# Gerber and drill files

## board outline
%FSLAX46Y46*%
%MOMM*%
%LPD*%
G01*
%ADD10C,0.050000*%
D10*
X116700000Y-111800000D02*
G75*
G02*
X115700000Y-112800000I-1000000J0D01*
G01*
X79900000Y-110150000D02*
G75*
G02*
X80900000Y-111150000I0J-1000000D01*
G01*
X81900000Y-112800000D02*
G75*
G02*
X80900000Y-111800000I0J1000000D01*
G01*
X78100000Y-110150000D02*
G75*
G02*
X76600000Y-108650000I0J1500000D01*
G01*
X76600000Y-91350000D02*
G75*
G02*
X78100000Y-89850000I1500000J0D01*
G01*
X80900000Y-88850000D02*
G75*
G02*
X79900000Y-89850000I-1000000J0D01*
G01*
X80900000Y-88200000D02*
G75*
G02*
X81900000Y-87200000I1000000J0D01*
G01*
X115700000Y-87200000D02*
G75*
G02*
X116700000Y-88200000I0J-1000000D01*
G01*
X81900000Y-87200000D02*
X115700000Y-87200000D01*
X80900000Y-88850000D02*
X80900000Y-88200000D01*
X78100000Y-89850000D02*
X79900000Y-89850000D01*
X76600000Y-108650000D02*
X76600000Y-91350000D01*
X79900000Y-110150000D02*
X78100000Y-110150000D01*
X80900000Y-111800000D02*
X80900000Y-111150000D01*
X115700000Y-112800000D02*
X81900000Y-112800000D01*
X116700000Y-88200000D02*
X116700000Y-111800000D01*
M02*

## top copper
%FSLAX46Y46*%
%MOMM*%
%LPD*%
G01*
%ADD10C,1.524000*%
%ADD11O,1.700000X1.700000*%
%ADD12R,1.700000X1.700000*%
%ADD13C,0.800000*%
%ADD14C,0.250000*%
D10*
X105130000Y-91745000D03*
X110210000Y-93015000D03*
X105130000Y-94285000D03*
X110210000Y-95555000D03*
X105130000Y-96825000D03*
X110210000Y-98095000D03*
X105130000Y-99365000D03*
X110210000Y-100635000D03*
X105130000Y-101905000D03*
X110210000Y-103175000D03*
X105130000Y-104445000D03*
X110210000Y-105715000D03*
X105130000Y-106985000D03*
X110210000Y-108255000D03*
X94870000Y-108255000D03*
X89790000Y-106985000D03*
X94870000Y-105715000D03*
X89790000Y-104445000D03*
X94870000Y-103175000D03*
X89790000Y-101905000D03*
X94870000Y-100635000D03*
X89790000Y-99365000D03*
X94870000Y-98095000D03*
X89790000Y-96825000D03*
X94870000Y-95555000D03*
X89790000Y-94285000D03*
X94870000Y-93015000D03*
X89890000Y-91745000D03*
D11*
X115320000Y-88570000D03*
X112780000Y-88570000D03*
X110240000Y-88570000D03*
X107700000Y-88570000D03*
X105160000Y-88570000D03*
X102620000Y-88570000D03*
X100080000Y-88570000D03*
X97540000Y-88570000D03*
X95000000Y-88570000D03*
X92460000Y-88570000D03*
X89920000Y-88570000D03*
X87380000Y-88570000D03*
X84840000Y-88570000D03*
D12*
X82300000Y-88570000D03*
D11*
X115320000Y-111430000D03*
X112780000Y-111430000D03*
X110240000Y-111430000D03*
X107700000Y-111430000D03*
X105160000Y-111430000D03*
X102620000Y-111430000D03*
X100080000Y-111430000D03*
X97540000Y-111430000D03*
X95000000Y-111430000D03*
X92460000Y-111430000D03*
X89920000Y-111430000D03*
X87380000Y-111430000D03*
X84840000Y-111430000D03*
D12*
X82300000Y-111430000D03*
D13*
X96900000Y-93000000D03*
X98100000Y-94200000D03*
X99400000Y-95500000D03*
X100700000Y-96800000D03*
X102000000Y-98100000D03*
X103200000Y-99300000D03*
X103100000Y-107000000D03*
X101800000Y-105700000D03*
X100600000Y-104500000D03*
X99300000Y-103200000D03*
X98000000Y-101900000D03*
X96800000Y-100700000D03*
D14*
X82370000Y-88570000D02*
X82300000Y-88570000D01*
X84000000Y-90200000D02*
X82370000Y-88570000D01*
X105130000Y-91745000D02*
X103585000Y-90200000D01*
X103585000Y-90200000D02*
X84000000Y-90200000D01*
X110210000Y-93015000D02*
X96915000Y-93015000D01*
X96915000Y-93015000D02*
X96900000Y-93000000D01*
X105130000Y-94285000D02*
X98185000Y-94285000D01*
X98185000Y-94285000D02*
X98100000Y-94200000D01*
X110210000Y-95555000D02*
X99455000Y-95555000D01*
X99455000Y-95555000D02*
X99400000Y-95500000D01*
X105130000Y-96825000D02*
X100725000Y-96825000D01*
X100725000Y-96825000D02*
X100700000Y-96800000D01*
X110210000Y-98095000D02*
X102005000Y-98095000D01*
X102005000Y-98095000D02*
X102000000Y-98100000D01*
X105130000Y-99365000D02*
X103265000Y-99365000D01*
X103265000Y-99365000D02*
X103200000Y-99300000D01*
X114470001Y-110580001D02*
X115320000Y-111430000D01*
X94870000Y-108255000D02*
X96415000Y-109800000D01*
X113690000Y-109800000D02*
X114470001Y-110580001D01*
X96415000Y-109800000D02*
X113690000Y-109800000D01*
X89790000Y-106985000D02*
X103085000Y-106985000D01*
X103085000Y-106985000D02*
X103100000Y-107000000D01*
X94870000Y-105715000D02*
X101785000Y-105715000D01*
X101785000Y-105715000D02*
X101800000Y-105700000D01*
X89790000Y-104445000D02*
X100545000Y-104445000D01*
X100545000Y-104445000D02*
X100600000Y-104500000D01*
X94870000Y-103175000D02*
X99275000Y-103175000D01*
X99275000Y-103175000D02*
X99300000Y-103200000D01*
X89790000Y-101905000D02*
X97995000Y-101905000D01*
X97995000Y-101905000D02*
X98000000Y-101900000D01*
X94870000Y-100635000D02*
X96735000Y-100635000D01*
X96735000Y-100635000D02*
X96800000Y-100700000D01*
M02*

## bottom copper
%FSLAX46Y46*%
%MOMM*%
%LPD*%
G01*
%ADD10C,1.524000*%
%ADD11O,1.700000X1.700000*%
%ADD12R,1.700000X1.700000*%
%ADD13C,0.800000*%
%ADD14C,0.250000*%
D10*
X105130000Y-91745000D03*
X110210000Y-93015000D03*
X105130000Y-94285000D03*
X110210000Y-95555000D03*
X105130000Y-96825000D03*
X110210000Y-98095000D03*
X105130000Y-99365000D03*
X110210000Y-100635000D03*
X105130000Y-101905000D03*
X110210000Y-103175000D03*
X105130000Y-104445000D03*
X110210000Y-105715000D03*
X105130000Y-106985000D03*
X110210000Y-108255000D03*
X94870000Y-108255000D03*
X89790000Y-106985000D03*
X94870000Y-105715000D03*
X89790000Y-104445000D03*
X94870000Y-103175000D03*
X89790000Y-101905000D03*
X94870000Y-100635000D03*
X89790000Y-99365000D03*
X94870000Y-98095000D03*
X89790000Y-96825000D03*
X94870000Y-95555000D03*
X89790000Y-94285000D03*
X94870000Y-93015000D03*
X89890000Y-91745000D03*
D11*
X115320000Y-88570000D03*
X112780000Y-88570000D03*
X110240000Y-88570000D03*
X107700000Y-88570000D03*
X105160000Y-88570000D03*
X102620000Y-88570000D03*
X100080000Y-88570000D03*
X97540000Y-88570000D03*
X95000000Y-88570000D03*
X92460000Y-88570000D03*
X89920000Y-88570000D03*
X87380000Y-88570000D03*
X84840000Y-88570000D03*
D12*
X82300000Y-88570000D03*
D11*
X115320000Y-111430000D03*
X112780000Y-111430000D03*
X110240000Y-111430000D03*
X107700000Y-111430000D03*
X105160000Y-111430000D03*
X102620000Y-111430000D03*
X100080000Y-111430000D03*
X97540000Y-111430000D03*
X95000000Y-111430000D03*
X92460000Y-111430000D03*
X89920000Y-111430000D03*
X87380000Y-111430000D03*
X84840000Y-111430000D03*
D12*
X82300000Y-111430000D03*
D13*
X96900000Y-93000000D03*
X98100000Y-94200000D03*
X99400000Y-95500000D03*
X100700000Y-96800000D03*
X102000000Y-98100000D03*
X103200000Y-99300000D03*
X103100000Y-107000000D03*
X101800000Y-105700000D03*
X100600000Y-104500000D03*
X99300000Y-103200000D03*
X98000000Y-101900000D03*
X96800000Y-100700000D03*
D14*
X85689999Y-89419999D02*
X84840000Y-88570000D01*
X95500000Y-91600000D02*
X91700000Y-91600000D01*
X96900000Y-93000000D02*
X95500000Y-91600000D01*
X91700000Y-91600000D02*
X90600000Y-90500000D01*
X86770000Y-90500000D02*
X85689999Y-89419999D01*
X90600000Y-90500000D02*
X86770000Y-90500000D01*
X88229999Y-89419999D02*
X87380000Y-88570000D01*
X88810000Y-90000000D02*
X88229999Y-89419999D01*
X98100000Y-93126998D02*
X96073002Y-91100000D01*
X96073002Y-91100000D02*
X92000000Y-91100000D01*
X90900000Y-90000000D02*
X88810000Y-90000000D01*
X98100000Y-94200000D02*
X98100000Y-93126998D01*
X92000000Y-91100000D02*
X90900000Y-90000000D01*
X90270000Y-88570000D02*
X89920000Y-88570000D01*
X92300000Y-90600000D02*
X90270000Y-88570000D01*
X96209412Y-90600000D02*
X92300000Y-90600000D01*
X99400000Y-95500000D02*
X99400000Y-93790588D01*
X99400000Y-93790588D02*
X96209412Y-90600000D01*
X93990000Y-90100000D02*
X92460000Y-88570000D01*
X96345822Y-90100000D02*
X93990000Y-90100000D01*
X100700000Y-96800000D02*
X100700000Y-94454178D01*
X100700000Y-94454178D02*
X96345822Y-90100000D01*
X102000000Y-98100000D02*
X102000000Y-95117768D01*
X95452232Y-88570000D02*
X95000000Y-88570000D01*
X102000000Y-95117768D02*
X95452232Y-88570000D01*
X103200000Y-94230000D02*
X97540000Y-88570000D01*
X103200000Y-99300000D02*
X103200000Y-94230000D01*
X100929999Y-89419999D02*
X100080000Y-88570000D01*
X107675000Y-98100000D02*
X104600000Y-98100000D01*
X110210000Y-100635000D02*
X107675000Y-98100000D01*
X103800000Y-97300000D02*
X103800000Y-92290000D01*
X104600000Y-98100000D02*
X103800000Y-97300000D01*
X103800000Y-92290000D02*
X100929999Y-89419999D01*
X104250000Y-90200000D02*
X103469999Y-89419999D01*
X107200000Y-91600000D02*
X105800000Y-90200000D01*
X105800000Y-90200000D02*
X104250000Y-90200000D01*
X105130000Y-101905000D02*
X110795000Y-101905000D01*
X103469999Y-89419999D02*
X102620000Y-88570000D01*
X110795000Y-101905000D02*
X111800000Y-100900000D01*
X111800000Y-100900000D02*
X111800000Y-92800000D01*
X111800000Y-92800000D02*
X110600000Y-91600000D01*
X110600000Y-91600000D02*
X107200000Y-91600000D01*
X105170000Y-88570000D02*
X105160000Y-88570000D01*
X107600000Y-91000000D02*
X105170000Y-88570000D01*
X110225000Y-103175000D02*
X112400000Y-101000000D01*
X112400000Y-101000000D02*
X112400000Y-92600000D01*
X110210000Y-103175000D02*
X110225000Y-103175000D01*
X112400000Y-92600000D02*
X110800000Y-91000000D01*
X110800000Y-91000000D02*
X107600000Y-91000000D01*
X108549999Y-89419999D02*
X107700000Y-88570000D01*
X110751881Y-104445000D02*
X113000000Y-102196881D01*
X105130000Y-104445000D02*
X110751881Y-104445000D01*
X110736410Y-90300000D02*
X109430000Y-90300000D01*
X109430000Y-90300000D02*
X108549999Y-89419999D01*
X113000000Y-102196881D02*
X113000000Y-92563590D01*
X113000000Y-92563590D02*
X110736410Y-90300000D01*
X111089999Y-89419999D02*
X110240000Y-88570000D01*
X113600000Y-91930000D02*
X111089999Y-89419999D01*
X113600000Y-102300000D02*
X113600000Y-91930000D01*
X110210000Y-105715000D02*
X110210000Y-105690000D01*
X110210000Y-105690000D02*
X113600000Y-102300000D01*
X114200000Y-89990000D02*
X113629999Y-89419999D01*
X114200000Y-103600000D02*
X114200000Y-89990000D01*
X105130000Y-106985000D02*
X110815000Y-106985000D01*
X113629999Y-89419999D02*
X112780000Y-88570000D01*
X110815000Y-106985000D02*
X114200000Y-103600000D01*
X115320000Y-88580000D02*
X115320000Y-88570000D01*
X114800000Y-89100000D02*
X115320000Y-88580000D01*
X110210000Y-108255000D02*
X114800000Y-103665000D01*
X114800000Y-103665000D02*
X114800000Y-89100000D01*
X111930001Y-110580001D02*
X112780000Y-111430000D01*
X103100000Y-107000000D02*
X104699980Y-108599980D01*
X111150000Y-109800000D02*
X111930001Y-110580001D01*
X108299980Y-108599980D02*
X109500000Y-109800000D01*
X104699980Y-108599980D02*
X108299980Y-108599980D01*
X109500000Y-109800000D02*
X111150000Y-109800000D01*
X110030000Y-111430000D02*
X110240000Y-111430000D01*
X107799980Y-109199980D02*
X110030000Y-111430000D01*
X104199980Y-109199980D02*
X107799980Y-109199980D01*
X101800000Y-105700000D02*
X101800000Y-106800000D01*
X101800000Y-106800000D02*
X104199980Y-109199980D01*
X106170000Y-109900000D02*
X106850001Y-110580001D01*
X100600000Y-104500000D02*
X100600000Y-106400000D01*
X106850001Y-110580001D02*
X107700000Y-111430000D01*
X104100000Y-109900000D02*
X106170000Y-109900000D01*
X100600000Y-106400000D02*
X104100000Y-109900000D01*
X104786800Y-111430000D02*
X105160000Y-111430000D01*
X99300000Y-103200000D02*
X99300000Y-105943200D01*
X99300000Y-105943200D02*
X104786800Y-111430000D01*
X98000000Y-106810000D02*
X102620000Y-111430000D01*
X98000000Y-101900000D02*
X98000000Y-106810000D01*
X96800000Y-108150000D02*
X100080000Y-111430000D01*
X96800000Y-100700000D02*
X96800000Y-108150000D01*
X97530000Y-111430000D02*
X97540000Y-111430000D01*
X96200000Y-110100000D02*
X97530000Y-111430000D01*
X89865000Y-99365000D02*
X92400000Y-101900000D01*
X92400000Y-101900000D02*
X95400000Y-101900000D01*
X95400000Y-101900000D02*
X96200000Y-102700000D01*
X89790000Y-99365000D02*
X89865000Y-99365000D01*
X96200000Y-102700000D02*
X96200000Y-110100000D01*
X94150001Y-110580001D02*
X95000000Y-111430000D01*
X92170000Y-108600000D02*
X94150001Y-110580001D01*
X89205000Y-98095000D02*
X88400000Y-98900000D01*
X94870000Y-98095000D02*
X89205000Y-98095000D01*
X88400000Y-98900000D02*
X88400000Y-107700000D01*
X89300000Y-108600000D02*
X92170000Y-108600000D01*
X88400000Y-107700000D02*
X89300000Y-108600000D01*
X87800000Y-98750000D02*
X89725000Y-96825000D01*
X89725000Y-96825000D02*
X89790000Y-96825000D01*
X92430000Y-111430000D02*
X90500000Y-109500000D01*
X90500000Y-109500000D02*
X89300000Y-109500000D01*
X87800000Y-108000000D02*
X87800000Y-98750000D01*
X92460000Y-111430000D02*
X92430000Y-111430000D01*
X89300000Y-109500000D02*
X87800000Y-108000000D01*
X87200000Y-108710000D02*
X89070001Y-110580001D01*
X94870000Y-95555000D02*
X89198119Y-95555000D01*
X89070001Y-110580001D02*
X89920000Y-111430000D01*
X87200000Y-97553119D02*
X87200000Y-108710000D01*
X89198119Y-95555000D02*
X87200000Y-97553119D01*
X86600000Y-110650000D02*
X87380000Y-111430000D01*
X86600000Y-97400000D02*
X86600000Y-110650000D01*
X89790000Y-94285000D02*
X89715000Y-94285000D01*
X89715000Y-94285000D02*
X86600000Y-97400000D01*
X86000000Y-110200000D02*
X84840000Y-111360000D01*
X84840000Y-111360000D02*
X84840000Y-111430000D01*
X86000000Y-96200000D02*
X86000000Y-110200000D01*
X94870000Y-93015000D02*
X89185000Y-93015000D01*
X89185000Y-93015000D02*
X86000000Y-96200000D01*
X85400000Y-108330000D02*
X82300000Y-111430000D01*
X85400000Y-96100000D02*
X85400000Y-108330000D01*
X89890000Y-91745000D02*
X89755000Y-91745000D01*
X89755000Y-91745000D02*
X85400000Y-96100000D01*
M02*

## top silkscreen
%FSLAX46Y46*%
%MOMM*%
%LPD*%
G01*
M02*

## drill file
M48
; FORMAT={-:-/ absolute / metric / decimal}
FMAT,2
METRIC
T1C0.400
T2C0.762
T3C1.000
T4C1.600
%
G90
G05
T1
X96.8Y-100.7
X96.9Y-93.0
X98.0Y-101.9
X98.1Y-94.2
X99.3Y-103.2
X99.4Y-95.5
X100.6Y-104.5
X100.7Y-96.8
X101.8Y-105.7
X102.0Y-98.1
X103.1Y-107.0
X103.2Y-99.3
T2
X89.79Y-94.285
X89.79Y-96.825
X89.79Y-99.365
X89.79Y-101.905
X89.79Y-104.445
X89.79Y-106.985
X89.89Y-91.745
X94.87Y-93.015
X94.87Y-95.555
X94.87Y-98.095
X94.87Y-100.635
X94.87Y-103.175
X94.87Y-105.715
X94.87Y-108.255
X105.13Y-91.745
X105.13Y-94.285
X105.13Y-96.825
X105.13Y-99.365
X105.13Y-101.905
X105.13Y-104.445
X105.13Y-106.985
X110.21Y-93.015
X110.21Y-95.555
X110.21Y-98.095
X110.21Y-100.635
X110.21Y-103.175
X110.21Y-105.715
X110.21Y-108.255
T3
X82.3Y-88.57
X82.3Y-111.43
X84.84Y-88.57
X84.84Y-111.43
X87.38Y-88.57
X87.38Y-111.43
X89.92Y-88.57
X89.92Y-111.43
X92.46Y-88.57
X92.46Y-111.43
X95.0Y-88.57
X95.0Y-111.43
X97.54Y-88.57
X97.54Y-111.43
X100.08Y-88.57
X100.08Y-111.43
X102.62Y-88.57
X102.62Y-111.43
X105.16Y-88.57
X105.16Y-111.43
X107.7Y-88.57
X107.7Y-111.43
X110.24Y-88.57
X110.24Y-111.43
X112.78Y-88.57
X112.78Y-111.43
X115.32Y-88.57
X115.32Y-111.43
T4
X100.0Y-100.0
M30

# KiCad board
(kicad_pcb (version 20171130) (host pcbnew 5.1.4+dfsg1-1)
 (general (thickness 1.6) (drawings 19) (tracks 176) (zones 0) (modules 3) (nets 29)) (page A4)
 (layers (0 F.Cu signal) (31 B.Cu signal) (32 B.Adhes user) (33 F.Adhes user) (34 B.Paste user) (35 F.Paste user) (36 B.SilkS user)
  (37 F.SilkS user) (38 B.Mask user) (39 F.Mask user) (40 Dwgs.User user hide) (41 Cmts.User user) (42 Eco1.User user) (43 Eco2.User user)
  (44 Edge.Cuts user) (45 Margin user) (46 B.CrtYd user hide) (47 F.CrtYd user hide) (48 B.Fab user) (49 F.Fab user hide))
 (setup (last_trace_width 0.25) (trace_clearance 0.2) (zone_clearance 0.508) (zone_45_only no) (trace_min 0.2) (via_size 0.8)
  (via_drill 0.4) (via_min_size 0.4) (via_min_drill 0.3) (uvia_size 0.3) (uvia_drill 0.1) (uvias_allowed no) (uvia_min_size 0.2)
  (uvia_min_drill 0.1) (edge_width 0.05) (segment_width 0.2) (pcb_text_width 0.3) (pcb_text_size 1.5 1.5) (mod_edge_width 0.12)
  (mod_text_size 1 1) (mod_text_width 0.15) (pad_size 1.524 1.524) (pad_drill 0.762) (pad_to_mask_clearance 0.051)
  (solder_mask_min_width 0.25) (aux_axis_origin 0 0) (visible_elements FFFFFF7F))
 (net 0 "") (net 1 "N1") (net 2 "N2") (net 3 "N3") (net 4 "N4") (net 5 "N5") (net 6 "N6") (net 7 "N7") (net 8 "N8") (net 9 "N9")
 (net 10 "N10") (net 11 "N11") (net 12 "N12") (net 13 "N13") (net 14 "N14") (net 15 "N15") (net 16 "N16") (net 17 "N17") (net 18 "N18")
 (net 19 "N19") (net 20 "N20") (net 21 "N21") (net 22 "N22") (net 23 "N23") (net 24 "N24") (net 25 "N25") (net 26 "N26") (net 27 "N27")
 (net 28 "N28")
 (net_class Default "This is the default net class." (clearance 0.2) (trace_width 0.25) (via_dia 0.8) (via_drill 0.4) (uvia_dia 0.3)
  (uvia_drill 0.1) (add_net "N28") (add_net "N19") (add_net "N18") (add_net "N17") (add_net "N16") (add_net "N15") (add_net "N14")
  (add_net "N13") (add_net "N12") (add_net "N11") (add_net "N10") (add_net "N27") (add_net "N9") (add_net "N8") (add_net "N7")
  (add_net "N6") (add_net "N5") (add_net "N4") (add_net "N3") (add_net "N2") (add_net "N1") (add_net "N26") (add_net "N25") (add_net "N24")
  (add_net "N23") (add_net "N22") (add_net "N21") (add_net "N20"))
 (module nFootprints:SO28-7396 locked (layer F.Cu) (at 100 100)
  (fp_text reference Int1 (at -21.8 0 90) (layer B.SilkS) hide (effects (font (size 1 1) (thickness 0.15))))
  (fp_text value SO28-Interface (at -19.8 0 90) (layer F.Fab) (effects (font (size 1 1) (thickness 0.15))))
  (pad "" np_thru_hole circle (at 0 0) (size 1.6 1.6) (drill 1.6) (layers *.Cu *.Mask))
  (pad 28 thru_hole circle (at 5.13 -8.255) (size 1.524 1.524) (drill 0.762) (layers *.Cu *.Mask) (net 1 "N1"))
  (pad 27 thru_hole circle (at 10.21 -6.985) (size 1.524 1.524) (drill 0.762) (layers *.Cu *.Mask) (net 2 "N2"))
  (pad 26 thru_hole circle (at 5.13 -5.715) (size 1.524 1.524) (drill 0.762) (layers *.Cu *.Mask) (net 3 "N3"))
  (pad 25 thru_hole circle (at 10.21 -4.445) (size 1.524 1.524) (drill 0.762) (layers *.Cu *.Mask) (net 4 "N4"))
  (pad 24 thru_hole circle (at 5.13 -3.175) (size 1.524 1.524) (drill 0.762) (layers *.Cu *.Mask) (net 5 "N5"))
  (pad 23 thru_hole circle (at 10.21 -1.905) (size 1.524 1.524) (drill 0.762) (layers *.Cu *.Mask) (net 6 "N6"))
  (pad 22 thru_hole circle (at 5.13 -0.635) (size 1.524 1.524) (drill 0.762) (layers *.Cu *.Mask) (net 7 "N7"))
  (pad 21 thru_hole circle (at 10.21 0.635) (size 1.524 1.524) (drill 0.762) (layers *.Cu *.Mask) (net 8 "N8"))
  (pad 20 thru_hole circle (at 5.13 1.905) (size 1.524 1.524) (drill 0.762) (layers *.Cu *.Mask) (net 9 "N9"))
  (pad 19 thru_hole circle (at 10.21 3.175) (size 1.524 1.524) (drill 0.762) (layers *.Cu *.Mask) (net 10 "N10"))
  (pad 18 thru_hole circle (at 5.13 4.445) (size 1.524 1.524) (drill 0.762) (layers *.Cu *.Mask) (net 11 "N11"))
  (pad 17 thru_hole circle (at 10.21 5.715) (size 1.524 1.524) (drill 0.762) (layers *.Cu *.Mask) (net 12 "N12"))
  (pad 16 thru_hole circle (at 5.13 6.985) (size 1.524 1.524) (drill 0.762) (layers *.Cu *.Mask) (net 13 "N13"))
  (pad 15 thru_hole circle (at 10.21 8.255) (size 1.524 1.524) (drill 0.762) (layers *.Cu *.Mask) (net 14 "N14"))
  (pad 14 thru_hole circle (at -5.13 8.255) (size 1.524 1.524) (drill 0.762) (layers *.Cu *.Mask) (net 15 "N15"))
  (pad 13 thru_hole circle (at -10.21 6.985) (size 1.524 1.524) (drill 0.762) (layers *.Cu *.Mask) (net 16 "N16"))
  (pad 12 thru_hole circle (at -5.13 5.715) (size 1.524 1.524) (drill 0.762) (layers *.Cu *.Mask) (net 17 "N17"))
  (pad 11 thru_hole circle (at -10.21 4.445) (size 1.524 1.524) (drill 0.762) (layers *.Cu *.Mask) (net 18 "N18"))
  (pad 10 thru_hole circle (at -5.13 3.175) (size 1.524 1.524) (drill 0.762) (layers *.Cu *.Mask) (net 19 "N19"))
  (pad 9 thru_hole circle (at -10.21 1.905) (size 1.524 1.524) (drill 0.762) (layers *.Cu *.Mask) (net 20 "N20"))
  (pad 8 thru_hole circle (at -5.13 0.635) (size 1.524 1.524) (drill 0.762) (layers *.Cu *.Mask) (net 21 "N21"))
  (pad 7 thru_hole circle (at -10.21 -0.635) (size 1.524 1.524) (drill 0.762) (layers *.Cu *.Mask) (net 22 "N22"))
  (pad 6 thru_hole circle (at -5.13 -1.905) (size 1.524 1.524) (drill 0.762) (layers *.Cu *.Mask) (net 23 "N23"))
  (pad 5 thru_hole circle (at -10.21 -3.175) (size 1.524 1.524) (drill 0.762) (layers *.Cu *.Mask) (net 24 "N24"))
  (pad 4 thru_hole circle (at -5.13 -4.445) (size 1.524 1.524) (drill 0.762) (layers *.Cu *.Mask) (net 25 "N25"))
  (pad 3 thru_hole circle (at -10.21 -5.715) (size 1.524 1.524) (drill 0.762) (layers *.Cu *.Mask) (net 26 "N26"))
  (pad 2 thru_hole circle (at -5.13 -6.985) (size 1.524 1.524) (drill 0.762) (layers *.Cu *.Mask) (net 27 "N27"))
  (pad 1 thru_hole circle (at -10.11 -8.255) (size 1.524 1.524) (drill 0.762) (layers *.Cu *.Mask) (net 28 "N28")))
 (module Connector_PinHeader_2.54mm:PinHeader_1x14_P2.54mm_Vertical (layer B.Cu) (at 82.3 88.57 270)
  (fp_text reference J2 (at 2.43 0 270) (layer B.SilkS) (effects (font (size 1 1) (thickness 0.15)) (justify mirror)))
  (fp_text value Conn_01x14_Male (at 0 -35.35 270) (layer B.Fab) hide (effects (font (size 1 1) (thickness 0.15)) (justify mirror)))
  (pad 14 thru_hole oval (at 0 -33.02 270) (size 1.7 1.7) (drill 1) (layers *.Cu *.Mask) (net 14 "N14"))
  (pad 13 thru_hole oval (at 0 -30.48 270) (size 1.7 1.7) (drill 1) (layers *.Cu *.Mask) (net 13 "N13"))
  (pad 12 thru_hole oval (at 0 -27.94 270) (size 1.7 1.7) (drill 1) (layers *.Cu *.Mask) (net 12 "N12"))
  (pad 11 thru_hole oval (at 0 -25.4 270) (size 1.7 1.7) (drill 1) (layers *.Cu *.Mask) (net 11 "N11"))
  (pad 10 thru_hole oval (at 0 -22.86 270) (size 1.7 1.7) (drill 1) (layers *.Cu *.Mask) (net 10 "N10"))
  (pad 9 thru_hole oval (at 0 -20.32 270) (size 1.7 1.7) (drill 1) (layers *.Cu *.Mask) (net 9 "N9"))
  (pad 8 thru_hole oval (at 0 -17.78 270) (size 1.7 1.7) (drill 1) (layers *.Cu *.Mask) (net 8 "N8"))
  (pad 7 thru_hole oval (at 0 -15.24 270) (size 1.7 1.7) (drill 1) (layers *.Cu *.Mask) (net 7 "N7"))
  (pad 6 thru_hole oval (at 0 -12.7 270) (size 1.7 1.7) (drill 1) (layers *.Cu *.Mask) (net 6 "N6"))
  (pad 5 thru_hole oval (at 0 -10.16 270) (size 1.7 1.7) (drill 1) (layers *.Cu *.Mask) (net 5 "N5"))
  (pad 4 thru_hole oval (at 0 -7.62 270) (size 1.7 1.7) (drill 1) (layers *.Cu *.Mask) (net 4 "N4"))
  (pad 3 thru_hole oval (at 0 -5.08 270) (size 1.7 1.7) (drill 1) (layers *.Cu *.Mask) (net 3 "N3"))
  (pad 2 thru_hole oval (at 0 -2.54 270) (size 1.7 1.7) (drill 1) (layers *.Cu *.Mask) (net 2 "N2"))
  (pad 1 thru_hole rect (at 0 0 270) (size 1.7 1.7) (drill 1) (layers *.Cu *.Mask) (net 1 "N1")))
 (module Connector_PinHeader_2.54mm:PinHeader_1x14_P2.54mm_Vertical (layer B.Cu) (at 82.3 111.43 270)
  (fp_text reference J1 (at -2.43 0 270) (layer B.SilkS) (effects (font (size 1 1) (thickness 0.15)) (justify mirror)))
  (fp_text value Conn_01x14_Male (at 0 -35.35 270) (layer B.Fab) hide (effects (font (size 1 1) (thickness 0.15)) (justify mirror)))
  (pad 14 thru_hole oval (at 0 -33.02 270) (size 1.7 1.7) (drill 1) (layers *.Cu *.Mask) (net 15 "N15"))
  (pad 13 thru_hole oval (at 0 -30.48 270) (size 1.7 1.7) (drill 1) (layers *.Cu *.Mask) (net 16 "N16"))
  (pad 12 thru_hole oval (at 0 -27.94 270) (size 1.7 1.7) (drill 1) (layers *.Cu *.Mask) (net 17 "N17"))
  (pad 11 thru_hole oval (at 0 -25.4 270) (size 1.7 1.7) (drill 1) (layers *.Cu *.Mask) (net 18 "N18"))
  (pad 10 thru_hole oval (at 0 -22.86 270) (size 1.7 1.7) (drill 1) (layers *.Cu *.Mask) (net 19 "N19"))
  (pad 9 thru_hole oval (at 0 -20.32 270) (size 1.7 1.7) (drill 1) (layers *.Cu *.Mask) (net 20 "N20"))
  (pad 8 thru_hole oval (at 0 -17.78 270) (size 1.7 1.7) (drill 1) (layers *.Cu *.Mask) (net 21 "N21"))
  (pad 7 thru_hole oval (at 0 -15.24 270) (size 1.7 1.7) (drill 1) (layers *.Cu *.Mask) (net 22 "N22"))
  (pad 6 thru_hole oval (at 0 -12.7 270) (size 1.7 1.7) (drill 1) (layers *.Cu *.Mask) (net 23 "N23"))
  (pad 5 thru_hole oval (at 0 -10.16 270) (size 1.7 1.7) (drill 1) (layers *.Cu *.Mask) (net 24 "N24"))
  (pad 4 thru_hole oval (at 0 -7.62 270) (size 1.7 1.7) (drill 1) (layers *.Cu *.Mask) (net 25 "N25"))
  (pad 3 thru_hole oval (at 0 -5.08 270) (size 1.7 1.7) (drill 1) (layers *.Cu *.Mask) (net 26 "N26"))
  (pad 2 thru_hole oval (at 0 -2.54 270) (size 1.7 1.7) (drill 1) (layers *.Cu *.Mask) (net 27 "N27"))
  (pad 1 thru_hole rect (at 0 0 270) (size 1.7 1.7) (drill 1) (layers *.Cu *.Mask) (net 28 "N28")))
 (gr_arc (start 115.7 111.8) (end 115.7 112.8) (angle -90) (layer Edge.Cuts) (width 0.05))
 (gr_arc (start 79.9 111.15) (end 80.9 111.15) (angle -90) (layer Edge.Cuts) (width 0.05))
 (gr_arc (start 81.9 111.8) (end 80.9 111.8) (angle -90) (layer Edge.Cuts) (width 0.05))
 (gr_arc (start 78.1 108.65) (end 76.6 108.65) (angle -90) (layer Edge.Cuts) (width 0.05))
 (gr_arc (start 78.1 91.35) (end 78.1 89.85) (angle -90) (layer Edge.Cuts) (width 0.05))
 (gr_arc (start 79.9 88.85) (end 79.9 89.85) (angle -90) (layer Edge.Cuts) (width 0.05))
 (gr_arc (start 81.9 88.2) (end 81.9 87.2) (angle -90) (layer Edge.Cuts) (width 0.05))
 (gr_arc (start 115.7 88.2) (end 116.7 88.2) (angle -90) (layer Edge.Cuts) (width 0.05))
 (gr_line (start 81.9 87.2) (end 115.7 87.2) (layer Edge.Cuts) (width 0.05))
 (gr_line (start 80.9 88.85) (end 80.9 88.2) (layer Edge.Cuts) (width 0.05))
 (gr_line (start 78.1 89.85) (end 79.9 89.85) (layer Edge.Cuts) (width 0.05))
 (gr_line (start 76.6 108.65) (end 76.6 91.35) (layer Edge.Cuts) (width 0.05))
 (gr_line (start 79.9 110.15) (end 78.1 110.15) (layer Edge.Cuts) (width 0.05))
 (gr_line (start 80.9 111.8) (end 80.9 111.15) (layer Edge.Cuts) (width 0.05))
 (gr_line (start 115.7 112.8) (end 81.9 112.8) (layer Edge.Cuts) (width 0.05))
 (gr_line (start 116.7 88.2) (end 116.7 111.8) (layer Edge.Cuts) (width 0.05))
 (segment (start 82.37 88.57) (end 82.3 88.57) (width 0.25) (layer F.Cu) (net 1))
 (segment (start 84 90.2) (end 82.37 88.57) (width 0.25) (layer F.Cu) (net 1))
 (segment (start 105.13 91.745) (end 103.585 90.2) (width 0.25) (layer F.Cu) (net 1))
 (segment (start 103.585 90.2) (end 84 90.2) (width 0.25) (layer F.Cu) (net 1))
 (via (at 96.9 93) (size 0.8) (drill 0.4) (layers F.Cu B.Cu) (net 2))
 (segment (start 110.21 93.015) (end 96.915 93.015) (width 0.25) (layer F.Cu) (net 2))
 (segment (start 96.915 93.015) (end 96.9 93) (width 0.25) (layer F.Cu) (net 2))
 (segment (start 85.689999 89.419999) (end 84.84 88.57) (width 0.25) (layer B.Cu) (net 2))
 (segment (start 95.5 91.6) (end 91.7 91.6) (width 0.25) (layer B.Cu) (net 2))
 (segment (start 96.9 93) (end 95.5 91.6) (width 0.25) (layer B.Cu) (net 2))
 (segment (start 91.7 91.6) (end 90.6 90.5) (width 0.25) (layer B.Cu) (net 2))
 (segment (start 86.77 90.5) (end 85.689999 89.419999) (width 0.25) (layer B.Cu) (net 2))
 (segment (start 90.6 90.5) (end 86.77 90.5) (width 0.25) (layer B.Cu) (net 2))
 (via (at 98.1 94.2) (size 0.8) (drill 0.4) (layers F.Cu B.Cu) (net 3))
 (segment (start 105.13 94.285) (end 98.185 94.285) (width 0.25) (layer F.Cu) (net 3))
 (segment (start 98.185 94.285) (end 98.1 94.2) (width 0.25) (layer F.Cu) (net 3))
 (segment (start 88.229999 89.419999) (end 87.38 88.57) (width 0.25) (layer B.Cu) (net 3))
 (segment (start 88.81 90) (end 88.229999 89.419999) (width 0.25) (layer B.Cu) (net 3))
 (segment (start 98.1 93.126998) (end 96.073002 91.1) (width 0.25) (layer B.Cu) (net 3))
 (segment (start 96.073002 91.1) (end 92 91.1) (width 0.25) (layer B.Cu) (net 3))
 (segment (start 90.9 90) (end 88.81 90) (width 0.25) (layer B.Cu) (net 3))
 (segment (start 98.1 94.2) (end 98.1 93.126998) (width 0.25) (layer B.Cu) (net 3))
 (segment (start 92 91.1) (end 90.9 90) (width 0.25) (layer B.Cu) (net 3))
 (segment (start 110.21 95.555) (end 99.455 95.555) (width 0.25) (layer F.Cu) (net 4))
 (via (at 99.4 95.5) (size 0.8) (drill 0.4) (layers F.Cu B.Cu) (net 4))
 (segment (start 99.455 95.555) (end 99.4 95.5) (width 0.25) (layer F.Cu) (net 4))
 (segment (start 90.27 88.57) (end 89.92 88.57) (width 0.25) (layer B.Cu) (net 4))
 (segment (start 92.3 90.6) (end 90.27 88.57) (width 0.25) (layer B.Cu) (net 4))
 (segment (start 96.209412 90.6) (end 92.3 90.6) (width 0.25) (layer B.Cu) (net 4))
 (segment (start 99.4 95.5) (end 99.4 93.790588) (width 0.25) (layer B.Cu) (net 4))
 (segment (start 99.4 93.790588) (end 96.209412 90.6) (width 0.25) (layer B.Cu) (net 4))
 (via (at 100.7 96.8) (size 0.8) (drill 0.4) (layers F.Cu B.Cu) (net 5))
 (segment (start 105.13 96.825) (end 100.725 96.825) (width 0.25) (layer F.Cu) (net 5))
 (segment (start 100.725 96.825) (end 100.7 96.8) (width 0.25) (layer F.Cu) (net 5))
 (segment (start 93.99 90.1) (end 92.46 88.57) (width 0.25) (layer B.Cu) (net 5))
 (segment (start 96.345822 90.1) (end 93.99 90.1) (width 0.25) (layer B.Cu) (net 5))
 (segment (start 100.7 96.8) (end 100.7 94.454178) (width 0.25) (layer B.Cu) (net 5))
 (segment (start 100.7 94.454178) (end 96.345822 90.1) (width 0.25) (layer B.Cu) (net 5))
 (via (at 102 98.1) (size 0.8) (drill 0.4) (layers F.Cu B.Cu) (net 6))
 (segment (start 110.21 98.095) (end 102.005 98.095) (width 0.25) (layer F.Cu) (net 6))
 (segment (start 102.005 98.095) (end 102 98.1) (width 0.25) (layer F.Cu) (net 6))
 (segment (start 102 98.1) (end 102 95.117768) (width 0.25) (layer B.Cu) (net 6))
 (segment (start 95.452232 88.57) (end 95 88.57) (width 0.25) (layer B.Cu) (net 6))
 (segment (start 102 95.117768) (end 95.452232 88.57) (width 0.25) (layer B.Cu) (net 6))
 (via (at 103.2 99.3) (size 0.8) (drill 0.4) (layers F.Cu B.Cu) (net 7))
 (segment (start 105.13 99.365) (end 103.265 99.365) (width 0.25) (layer F.Cu) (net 7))
 (segment (start 103.265 99.365) (end 103.2 99.3) (width 0.25) (layer F.Cu) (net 7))
 (segment (start 103.2 94.23) (end 97.54 88.57) (width 0.25) (layer B.Cu) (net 7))
 (segment (start 103.2 99.3) (end 103.2 94.23) (width 0.25) (layer B.Cu) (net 7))
 (segment (start 100.929999 89.419999) (end 100.08 88.57) (width 0.25) (layer B.Cu) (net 8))
 (segment (start 107.675 98.1) (end 104.6 98.1) (width 0.25) (layer B.Cu) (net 8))
 (segment (start 110.21 100.635) (end 107.675 98.1) (width 0.25) (layer B.Cu) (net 8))
 (segment (start 103.8 97.3) (end 103.8 92.29) (width 0.25) (layer B.Cu) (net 8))
 (segment (start 104.6 98.1) (end 103.8 97.3) (width 0.25) (layer B.Cu) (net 8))
 (segment (start 103.8 92.29) (end 100.929999 89.419999) (width 0.25) (layer B.Cu) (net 8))
 (segment (start 104.25 90.2) (end 103.469999 89.419999) (width 0.25) (layer B.Cu) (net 9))
 (segment (start 107.2 91.6) (end 105.8 90.2) (width 0.25) (layer B.Cu) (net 9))
 (segment (start 105.8 90.2) (end 104.25 90.2) (width 0.25) (layer B.Cu) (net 9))
 (segment (start 105.13 101.905) (end 110.795 101.905) (width 0.25) (layer B.Cu) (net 9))
 (segment (start 103.469999 89.419999) (end 102.62 88.57) (width 0.25) (layer B.Cu) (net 9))
 (segment (start 110.795 101.905) (end 111.8 100.9) (width 0.25) (layer B.Cu) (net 9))
 (segment (start 111.8 100.9) (end 111.8 92.8) (width 0.25) (layer B.Cu) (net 9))
 (segment (start 111.8 92.8) (end 110.6 91.6) (width 0.25) (layer B.Cu) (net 9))
 (segment (start 110.6 91.6) (end 107.2 91.6) (width 0.25) (layer B.Cu) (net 9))
 (segment (start 105.17 88.57) (end 105.16 88.57) (width 0.25) (layer B.Cu) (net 10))
 (segment (start 107.6 91) (end 105.17 88.57) (width 0.25) (layer B.Cu) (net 10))
 (segment (start 110.225 103.175) (end 112.4 101) (width 0.25) (layer B.Cu) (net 10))
 (segment (start 112.4 101) (end 112.4 92.6) (width 0.25) (layer B.Cu) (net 10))
 (segment (start 110.21 103.175) (end 110.225 103.175) (width 0.25) (layer B.Cu) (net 10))
 (segment (start 112.4 92.6) (end 110.8 91) (width 0.25) (layer B.Cu) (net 10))
 (segment (start 110.8 91) (end 107.6 91) (width 0.25) (layer B.Cu) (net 10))
 (segment (start 108.549999 89.419999) (end 107.7 88.57) (width 0.25) (layer B.Cu) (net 11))
 (segment (start 110.751881 104.445) (end 113 102.196881) (width 0.25) (layer B.Cu) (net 11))
 (segment (start 105.13 104.445) (end 110.751881 104.445) (width 0.25) (layer B.Cu) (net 11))
 (segment (start 110.73641 90.3) (end 109.43 90.3) (width 0.25) (layer B.Cu) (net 11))
 (segment (start 109.43 90.3) (end 108.549999 89.419999) (width 0.25) (layer B.Cu) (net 11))
 (segment (start 113 102.196881) (end 113 92.56359) (width 0.25) (layer B.Cu) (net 11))
 (segment (start 113 92.56359) (end 110.73641 90.3) (width 0.25) (layer B.Cu) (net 11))
 (segment (start 111.089999 89.419999) (end 110.24 88.57) (width 0.25) (layer B.Cu) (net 12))
 (segment (start 113.6 91.93) (end 111.089999 89.419999) (width 0.25) (layer B.Cu) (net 12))
 (segment (start 113.6 102.3) (end 113.6 91.93) (width 0.25) (layer B.Cu) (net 12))
 (segment (start 110.21 105.715) (end 110.21 105.69) (width 0.25) (layer B.Cu) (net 12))
 (segment (start 110.21 105.69) (end 113.6 102.3) (width 0.25) (layer B.Cu) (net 12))
 (segment (start 114.2 89.99) (end 113.629999 89.419999) (width 0.25) (layer B.Cu) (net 13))
 (segment (start 114.2 103.6) (end 114.2 89.99) (width 0.25) (layer B.Cu) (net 13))
 (segment (start 105.13 106.985) (end 110.815 106.985) (width 0.25) (layer B.Cu) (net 13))
 (segment (start 113.629999 89.419999) (end 112.78 88.57) (width 0.25) (layer B.Cu) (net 13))
 (segment (start 110.815 106.985) (end 114.2 103.6) (width 0.25) (layer B.Cu) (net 13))
 (segment (start 115.32 88.58) (end 115.32 88.57) (width 0.25) (layer B.Cu) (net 14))
 (segment (start 114.8 89.1) (end 115.32 88.58) (width 0.25) (layer B.Cu) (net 14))
 (segment (start 110.21 108.255) (end 114.8 103.665) (width 0.25) (layer B.Cu) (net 14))
 (segment (start 114.8 103.665) (end 114.8 89.1) (width 0.25) (layer B.Cu) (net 14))
 (segment (start 114.470001 110.580001) (end 115.32 111.43) (width 0.25) (layer F.Cu) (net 15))
 (segment (start 94.87 108.255) (end 96.415 109.8) (width 0.25) (layer F.Cu) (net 15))
 (segment (start 113.69 109.8) (end 114.470001 110.580001) (width 0.25) (layer F.Cu) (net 15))
 (segment (start 96.415 109.8) (end 113.69 109.8) (width 0.25) (layer F.Cu) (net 15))
 (via (at 103.1 107) (size 0.8) (drill 0.4) (layers F.Cu B.Cu) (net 16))
 (segment (start 89.79 106.985) (end 103.085 106.985) (width 0.25) (layer F.Cu) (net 16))
 (segment (start 103.085 106.985) (end 103.1 107) (width 0.25) (layer F.Cu) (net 16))
 (segment (start 111.930001 110.580001) (end 112.78 111.43) (width 0.25) (layer B.Cu) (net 16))
 (segment (start 103.1 107) (end 104.69998 108.59998) (width 0.25) (layer B.Cu) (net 16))
 (segment (start 111.15 109.8) (end 111.930001 110.580001) (width 0.25) (layer B.Cu) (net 16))
 (segment (start 108.29998 108.59998) (end 109.5 109.8) (width 0.25) (layer B.Cu) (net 16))
 (segment (start 104.69998 108.59998) (end 108.29998 108.59998) (width 0.25) (layer B.Cu) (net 16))
 (segment (start 109.5 109.8) (end 111.15 109.8) (width 0.25) (layer B.Cu) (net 16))
 (via (at 101.8 105.7) (size 0.8) (drill 0.4) (layers F.Cu B.Cu) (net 17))
 (segment (start 94.87 105.715) (end 101.785 105.715) (width 0.25) (layer F.Cu) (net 17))
 (segment (start 101.785 105.715) (end 101.8 105.7) (width 0.25) (layer F.Cu) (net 17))
 (segment (start 110.03 111.43) (end 110.24 111.43) (width 0.25) (layer B.Cu) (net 17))
 (segment (start 107.79998 109.19998) (end 110.03 111.43) (width 0.25) (layer B.Cu) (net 17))
 (segment (start 104.19998 109.19998) (end 107.79998 109.19998) (width 0.25) (layer B.Cu) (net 17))
 (segment (start 101.8 105.7) (end 101.8 106.8) (width 0.25) (layer B.Cu) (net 17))
 (segment (start 101.8 106.8) (end 104.19998 109.19998) (width 0.25) (layer B.Cu) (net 17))
 (via (at 100.6 104.5) (size 0.8) (drill 0.4) (layers F.Cu B.Cu) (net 18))
 (segment (start 89.79 104.445) (end 100.545 104.445) (width 0.25) (layer F.Cu) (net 18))
 (segment (start 100.545 104.445) (end 100.6 104.5) (width 0.25) (layer F.Cu) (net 18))
 (segment (start 106.17 109.9) (end 106.850001 110.580001) (width 0.25) (layer B.Cu) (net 18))
 (segment (start 100.6 104.5) (end 100.6 106.4) (width 0.25) (layer B.Cu) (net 18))
 (segment (start 106.850001 110.580001) (end 107.7 111.43) (width 0.25) (layer B.Cu) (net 18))
 (segment (start 104.1 109.9) (end 106.17 109.9) (width 0.25) (layer B.Cu) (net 18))
 (segment (start 100.6 106.4) (end 104.1 109.9) (width 0.25) (layer B.Cu) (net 18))
 (via (at 99.3 103.2) (size 0.8) (drill 0.4) (layers F.Cu B.Cu) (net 19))
 (segment (start 94.87 103.175) (end 99.275 103.175) (width 0.25) (layer F.Cu) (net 19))
 (segment (start 99.275 103.175) (end 99.3 103.2) (width 0.25) (layer F.Cu) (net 19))
 (segment (start 104.7868 111.43) (end 105.16 111.43) (width 0.25) (layer B.Cu) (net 19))
 (segment (start 99.3 103.2) (end 99.3 105.9432) (width 0.25) (layer B.Cu) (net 19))
 (segment (start 99.3 105.9432) (end 104.7868 111.43) (width 0.25) (layer B.Cu) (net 19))
 (segment (start 89.79 101.905) (end 97.995 101.905) (width 0.25) (layer F.Cu) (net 20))
 (via (at 98 101.9) (size 0.8) (drill 0.4) (layers F.Cu B.Cu) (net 20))
 (segment (start 97.995 101.905) (end 98 101.9) (width 0.25) (layer F.Cu) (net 20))
 (segment (start 98 106.81) (end 102.62 111.43) (width 0.25) (layer B.Cu) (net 20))
 (segment (start 98 101.9) (end 98 106.81) (width 0.25) (layer B.Cu) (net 20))
 (via (at 96.8 100.7) (size 0.8) (drill 0.4) (layers F.Cu B.Cu) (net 21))
 (segment (start 94.87 100.635) (end 96.735 100.635) (width 0.25) (layer F.Cu) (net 21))
 (segment (start 96.735 100.635) (end 96.8 100.7) (width 0.25) (layer F.Cu) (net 21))
 (segment (start 96.8 108.15) (end 100.08 111.43) (width 0.25) (layer B.Cu) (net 21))
 (segment (start 96.8 100.7) (end 96.8 108.15) (width 0.25) (layer B.Cu) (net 21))
 (segment (start 97.53 111.43) (end 97.54 111.43) (width 0.25) (layer B.Cu) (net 22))
 (segment (start 96.2 110.1) (end 97.53 111.43) (width 0.25) (layer B.Cu) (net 22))
 (segment (start 89.865 99.365) (end 92.4 101.9) (width 0.25) (layer B.Cu) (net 22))
 (segment (start 92.4 101.9) (end 95.4 101.9) (width 0.25) (layer B.Cu) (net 22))
 (segment (start 95.4 101.9) (end 96.2 102.7) (width 0.25) (layer B.Cu) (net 22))
 (segment (start 89.79 99.365) (end 89.865 99.365) (width 0.25) (layer B.Cu) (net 22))
 (segment (start 96.2 102.7) (end 96.2 110.1) (width 0.25) (layer B.Cu) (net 22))
 (segment (start 94.150001 110.580001) (end 95 111.43) (width 0.25) (layer B.Cu) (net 23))
 (segment (start 92.17 108.6) (end 94.150001 110.580001) (width 0.25) (layer B.Cu) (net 23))
 (segment (start 89.205 98.095) (end 88.4 98.9) (width 0.25) (layer B.Cu) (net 23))
 (segment (start 94.87 98.095) (end 89.205 98.095) (width 0.25) (layer B.Cu) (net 23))
 (segment (start 88.4 98.9) (end 88.4 107.7) (width 0.25) (layer B.Cu) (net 23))
 (segment (start 89.3 108.6) (end 92.17 108.6) (width 0.25) (layer B.Cu) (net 23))
 (segment (start 88.4 107.7) (end 89.3 108.6) (width 0.25) (layer B.Cu) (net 23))
 (segment (start 87.8 98.75) (end 89.725 96.825) (width 0.25) (layer B.Cu) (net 24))
 (segment (start 89.725 96.825) (end 89.79 96.825) (width 0.25) (layer B.Cu) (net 24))
 (segment (start 92.43 111.43) (end 90.5 109.5) (width 0.25) (layer B.Cu) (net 24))
 (segment (start 90.5 109.5) (end 89.3 109.5) (width 0.25) (layer B.Cu) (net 24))
 (segment (start 87.8 108) (end 87.8 98.75) (width 0.25) (layer B.Cu) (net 24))
 (segment (start 92.46 111.43) (end 92.43 111.43) (width 0.25) (layer B.Cu) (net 24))
 (segment (start 89.3 109.5) (end 87.8 108) (width 0.25) (layer B.Cu) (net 24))
 (segment (start 87.2 108.71) (end 89.070001 110.580001) (width 0.25) (layer B.Cu) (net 25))
 (segment (start 94.87 95.555) (end 89.198119 95.555) (width 0.25) (layer B.Cu) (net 25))
 (segment (start 89.070001 110.580001) (end 89.92 111.43) (width 0.25) (layer B.Cu) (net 25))
 (segment (start 87.2 97.553119) (end 87.2 108.71) (width 0.25) (layer B.Cu) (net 25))
 (segment (start 89.198119 95.555) (end 87.2 97.553119) (width 0.25) (layer B.Cu) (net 25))
 (segment (start 86.6 110.65) (end 87.38 111.43) (width 0.25) (layer B.Cu) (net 26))
 (segment (start 86.6 97.4) (end 86.6 110.65) (width 0.25) (layer B.Cu) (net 26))
 (segment (start 89.79 94.285) (end 89.715 94.285) (width 0.25) (layer B.Cu) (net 26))
 (segment (start 89.715 94.285) (end 86.6 97.4) (width 0.25) (layer B.Cu) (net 26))
 (segment (start 86 110.2) (end 84.84 111.36) (width 0.25) (layer B.Cu) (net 27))
 (segment (start 84.84 111.36) (end 84.84 111.43) (width 0.25) (layer B.Cu) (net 27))
 (segment (start 86 96.2) (end 86 110.2) (width 0.25) (layer B.Cu) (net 27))
 (segment (start 94.87 93.015) (end 89.185 93.015) (width 0.25) (layer B.Cu) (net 27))
 (segment (start 89.185 93.015) (end 86 96.2) (width 0.25) (layer B.Cu) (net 27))
 (segment (start 85.4 108.33) (end 82.3 111.43) (width 0.25) (layer B.Cu) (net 28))
 (segment (start 85.4 96.1) (end 85.4 108.33) (width 0.25) (layer B.Cu) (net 28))
 (segment (start 89.89 91.745) (end 89.755 91.745) (width 0.25) (layer B.Cu) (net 28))
 (segment (start 89.755 91.745) (end 85.4 96.1) (width 0.25) (layer B.Cu) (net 28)))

